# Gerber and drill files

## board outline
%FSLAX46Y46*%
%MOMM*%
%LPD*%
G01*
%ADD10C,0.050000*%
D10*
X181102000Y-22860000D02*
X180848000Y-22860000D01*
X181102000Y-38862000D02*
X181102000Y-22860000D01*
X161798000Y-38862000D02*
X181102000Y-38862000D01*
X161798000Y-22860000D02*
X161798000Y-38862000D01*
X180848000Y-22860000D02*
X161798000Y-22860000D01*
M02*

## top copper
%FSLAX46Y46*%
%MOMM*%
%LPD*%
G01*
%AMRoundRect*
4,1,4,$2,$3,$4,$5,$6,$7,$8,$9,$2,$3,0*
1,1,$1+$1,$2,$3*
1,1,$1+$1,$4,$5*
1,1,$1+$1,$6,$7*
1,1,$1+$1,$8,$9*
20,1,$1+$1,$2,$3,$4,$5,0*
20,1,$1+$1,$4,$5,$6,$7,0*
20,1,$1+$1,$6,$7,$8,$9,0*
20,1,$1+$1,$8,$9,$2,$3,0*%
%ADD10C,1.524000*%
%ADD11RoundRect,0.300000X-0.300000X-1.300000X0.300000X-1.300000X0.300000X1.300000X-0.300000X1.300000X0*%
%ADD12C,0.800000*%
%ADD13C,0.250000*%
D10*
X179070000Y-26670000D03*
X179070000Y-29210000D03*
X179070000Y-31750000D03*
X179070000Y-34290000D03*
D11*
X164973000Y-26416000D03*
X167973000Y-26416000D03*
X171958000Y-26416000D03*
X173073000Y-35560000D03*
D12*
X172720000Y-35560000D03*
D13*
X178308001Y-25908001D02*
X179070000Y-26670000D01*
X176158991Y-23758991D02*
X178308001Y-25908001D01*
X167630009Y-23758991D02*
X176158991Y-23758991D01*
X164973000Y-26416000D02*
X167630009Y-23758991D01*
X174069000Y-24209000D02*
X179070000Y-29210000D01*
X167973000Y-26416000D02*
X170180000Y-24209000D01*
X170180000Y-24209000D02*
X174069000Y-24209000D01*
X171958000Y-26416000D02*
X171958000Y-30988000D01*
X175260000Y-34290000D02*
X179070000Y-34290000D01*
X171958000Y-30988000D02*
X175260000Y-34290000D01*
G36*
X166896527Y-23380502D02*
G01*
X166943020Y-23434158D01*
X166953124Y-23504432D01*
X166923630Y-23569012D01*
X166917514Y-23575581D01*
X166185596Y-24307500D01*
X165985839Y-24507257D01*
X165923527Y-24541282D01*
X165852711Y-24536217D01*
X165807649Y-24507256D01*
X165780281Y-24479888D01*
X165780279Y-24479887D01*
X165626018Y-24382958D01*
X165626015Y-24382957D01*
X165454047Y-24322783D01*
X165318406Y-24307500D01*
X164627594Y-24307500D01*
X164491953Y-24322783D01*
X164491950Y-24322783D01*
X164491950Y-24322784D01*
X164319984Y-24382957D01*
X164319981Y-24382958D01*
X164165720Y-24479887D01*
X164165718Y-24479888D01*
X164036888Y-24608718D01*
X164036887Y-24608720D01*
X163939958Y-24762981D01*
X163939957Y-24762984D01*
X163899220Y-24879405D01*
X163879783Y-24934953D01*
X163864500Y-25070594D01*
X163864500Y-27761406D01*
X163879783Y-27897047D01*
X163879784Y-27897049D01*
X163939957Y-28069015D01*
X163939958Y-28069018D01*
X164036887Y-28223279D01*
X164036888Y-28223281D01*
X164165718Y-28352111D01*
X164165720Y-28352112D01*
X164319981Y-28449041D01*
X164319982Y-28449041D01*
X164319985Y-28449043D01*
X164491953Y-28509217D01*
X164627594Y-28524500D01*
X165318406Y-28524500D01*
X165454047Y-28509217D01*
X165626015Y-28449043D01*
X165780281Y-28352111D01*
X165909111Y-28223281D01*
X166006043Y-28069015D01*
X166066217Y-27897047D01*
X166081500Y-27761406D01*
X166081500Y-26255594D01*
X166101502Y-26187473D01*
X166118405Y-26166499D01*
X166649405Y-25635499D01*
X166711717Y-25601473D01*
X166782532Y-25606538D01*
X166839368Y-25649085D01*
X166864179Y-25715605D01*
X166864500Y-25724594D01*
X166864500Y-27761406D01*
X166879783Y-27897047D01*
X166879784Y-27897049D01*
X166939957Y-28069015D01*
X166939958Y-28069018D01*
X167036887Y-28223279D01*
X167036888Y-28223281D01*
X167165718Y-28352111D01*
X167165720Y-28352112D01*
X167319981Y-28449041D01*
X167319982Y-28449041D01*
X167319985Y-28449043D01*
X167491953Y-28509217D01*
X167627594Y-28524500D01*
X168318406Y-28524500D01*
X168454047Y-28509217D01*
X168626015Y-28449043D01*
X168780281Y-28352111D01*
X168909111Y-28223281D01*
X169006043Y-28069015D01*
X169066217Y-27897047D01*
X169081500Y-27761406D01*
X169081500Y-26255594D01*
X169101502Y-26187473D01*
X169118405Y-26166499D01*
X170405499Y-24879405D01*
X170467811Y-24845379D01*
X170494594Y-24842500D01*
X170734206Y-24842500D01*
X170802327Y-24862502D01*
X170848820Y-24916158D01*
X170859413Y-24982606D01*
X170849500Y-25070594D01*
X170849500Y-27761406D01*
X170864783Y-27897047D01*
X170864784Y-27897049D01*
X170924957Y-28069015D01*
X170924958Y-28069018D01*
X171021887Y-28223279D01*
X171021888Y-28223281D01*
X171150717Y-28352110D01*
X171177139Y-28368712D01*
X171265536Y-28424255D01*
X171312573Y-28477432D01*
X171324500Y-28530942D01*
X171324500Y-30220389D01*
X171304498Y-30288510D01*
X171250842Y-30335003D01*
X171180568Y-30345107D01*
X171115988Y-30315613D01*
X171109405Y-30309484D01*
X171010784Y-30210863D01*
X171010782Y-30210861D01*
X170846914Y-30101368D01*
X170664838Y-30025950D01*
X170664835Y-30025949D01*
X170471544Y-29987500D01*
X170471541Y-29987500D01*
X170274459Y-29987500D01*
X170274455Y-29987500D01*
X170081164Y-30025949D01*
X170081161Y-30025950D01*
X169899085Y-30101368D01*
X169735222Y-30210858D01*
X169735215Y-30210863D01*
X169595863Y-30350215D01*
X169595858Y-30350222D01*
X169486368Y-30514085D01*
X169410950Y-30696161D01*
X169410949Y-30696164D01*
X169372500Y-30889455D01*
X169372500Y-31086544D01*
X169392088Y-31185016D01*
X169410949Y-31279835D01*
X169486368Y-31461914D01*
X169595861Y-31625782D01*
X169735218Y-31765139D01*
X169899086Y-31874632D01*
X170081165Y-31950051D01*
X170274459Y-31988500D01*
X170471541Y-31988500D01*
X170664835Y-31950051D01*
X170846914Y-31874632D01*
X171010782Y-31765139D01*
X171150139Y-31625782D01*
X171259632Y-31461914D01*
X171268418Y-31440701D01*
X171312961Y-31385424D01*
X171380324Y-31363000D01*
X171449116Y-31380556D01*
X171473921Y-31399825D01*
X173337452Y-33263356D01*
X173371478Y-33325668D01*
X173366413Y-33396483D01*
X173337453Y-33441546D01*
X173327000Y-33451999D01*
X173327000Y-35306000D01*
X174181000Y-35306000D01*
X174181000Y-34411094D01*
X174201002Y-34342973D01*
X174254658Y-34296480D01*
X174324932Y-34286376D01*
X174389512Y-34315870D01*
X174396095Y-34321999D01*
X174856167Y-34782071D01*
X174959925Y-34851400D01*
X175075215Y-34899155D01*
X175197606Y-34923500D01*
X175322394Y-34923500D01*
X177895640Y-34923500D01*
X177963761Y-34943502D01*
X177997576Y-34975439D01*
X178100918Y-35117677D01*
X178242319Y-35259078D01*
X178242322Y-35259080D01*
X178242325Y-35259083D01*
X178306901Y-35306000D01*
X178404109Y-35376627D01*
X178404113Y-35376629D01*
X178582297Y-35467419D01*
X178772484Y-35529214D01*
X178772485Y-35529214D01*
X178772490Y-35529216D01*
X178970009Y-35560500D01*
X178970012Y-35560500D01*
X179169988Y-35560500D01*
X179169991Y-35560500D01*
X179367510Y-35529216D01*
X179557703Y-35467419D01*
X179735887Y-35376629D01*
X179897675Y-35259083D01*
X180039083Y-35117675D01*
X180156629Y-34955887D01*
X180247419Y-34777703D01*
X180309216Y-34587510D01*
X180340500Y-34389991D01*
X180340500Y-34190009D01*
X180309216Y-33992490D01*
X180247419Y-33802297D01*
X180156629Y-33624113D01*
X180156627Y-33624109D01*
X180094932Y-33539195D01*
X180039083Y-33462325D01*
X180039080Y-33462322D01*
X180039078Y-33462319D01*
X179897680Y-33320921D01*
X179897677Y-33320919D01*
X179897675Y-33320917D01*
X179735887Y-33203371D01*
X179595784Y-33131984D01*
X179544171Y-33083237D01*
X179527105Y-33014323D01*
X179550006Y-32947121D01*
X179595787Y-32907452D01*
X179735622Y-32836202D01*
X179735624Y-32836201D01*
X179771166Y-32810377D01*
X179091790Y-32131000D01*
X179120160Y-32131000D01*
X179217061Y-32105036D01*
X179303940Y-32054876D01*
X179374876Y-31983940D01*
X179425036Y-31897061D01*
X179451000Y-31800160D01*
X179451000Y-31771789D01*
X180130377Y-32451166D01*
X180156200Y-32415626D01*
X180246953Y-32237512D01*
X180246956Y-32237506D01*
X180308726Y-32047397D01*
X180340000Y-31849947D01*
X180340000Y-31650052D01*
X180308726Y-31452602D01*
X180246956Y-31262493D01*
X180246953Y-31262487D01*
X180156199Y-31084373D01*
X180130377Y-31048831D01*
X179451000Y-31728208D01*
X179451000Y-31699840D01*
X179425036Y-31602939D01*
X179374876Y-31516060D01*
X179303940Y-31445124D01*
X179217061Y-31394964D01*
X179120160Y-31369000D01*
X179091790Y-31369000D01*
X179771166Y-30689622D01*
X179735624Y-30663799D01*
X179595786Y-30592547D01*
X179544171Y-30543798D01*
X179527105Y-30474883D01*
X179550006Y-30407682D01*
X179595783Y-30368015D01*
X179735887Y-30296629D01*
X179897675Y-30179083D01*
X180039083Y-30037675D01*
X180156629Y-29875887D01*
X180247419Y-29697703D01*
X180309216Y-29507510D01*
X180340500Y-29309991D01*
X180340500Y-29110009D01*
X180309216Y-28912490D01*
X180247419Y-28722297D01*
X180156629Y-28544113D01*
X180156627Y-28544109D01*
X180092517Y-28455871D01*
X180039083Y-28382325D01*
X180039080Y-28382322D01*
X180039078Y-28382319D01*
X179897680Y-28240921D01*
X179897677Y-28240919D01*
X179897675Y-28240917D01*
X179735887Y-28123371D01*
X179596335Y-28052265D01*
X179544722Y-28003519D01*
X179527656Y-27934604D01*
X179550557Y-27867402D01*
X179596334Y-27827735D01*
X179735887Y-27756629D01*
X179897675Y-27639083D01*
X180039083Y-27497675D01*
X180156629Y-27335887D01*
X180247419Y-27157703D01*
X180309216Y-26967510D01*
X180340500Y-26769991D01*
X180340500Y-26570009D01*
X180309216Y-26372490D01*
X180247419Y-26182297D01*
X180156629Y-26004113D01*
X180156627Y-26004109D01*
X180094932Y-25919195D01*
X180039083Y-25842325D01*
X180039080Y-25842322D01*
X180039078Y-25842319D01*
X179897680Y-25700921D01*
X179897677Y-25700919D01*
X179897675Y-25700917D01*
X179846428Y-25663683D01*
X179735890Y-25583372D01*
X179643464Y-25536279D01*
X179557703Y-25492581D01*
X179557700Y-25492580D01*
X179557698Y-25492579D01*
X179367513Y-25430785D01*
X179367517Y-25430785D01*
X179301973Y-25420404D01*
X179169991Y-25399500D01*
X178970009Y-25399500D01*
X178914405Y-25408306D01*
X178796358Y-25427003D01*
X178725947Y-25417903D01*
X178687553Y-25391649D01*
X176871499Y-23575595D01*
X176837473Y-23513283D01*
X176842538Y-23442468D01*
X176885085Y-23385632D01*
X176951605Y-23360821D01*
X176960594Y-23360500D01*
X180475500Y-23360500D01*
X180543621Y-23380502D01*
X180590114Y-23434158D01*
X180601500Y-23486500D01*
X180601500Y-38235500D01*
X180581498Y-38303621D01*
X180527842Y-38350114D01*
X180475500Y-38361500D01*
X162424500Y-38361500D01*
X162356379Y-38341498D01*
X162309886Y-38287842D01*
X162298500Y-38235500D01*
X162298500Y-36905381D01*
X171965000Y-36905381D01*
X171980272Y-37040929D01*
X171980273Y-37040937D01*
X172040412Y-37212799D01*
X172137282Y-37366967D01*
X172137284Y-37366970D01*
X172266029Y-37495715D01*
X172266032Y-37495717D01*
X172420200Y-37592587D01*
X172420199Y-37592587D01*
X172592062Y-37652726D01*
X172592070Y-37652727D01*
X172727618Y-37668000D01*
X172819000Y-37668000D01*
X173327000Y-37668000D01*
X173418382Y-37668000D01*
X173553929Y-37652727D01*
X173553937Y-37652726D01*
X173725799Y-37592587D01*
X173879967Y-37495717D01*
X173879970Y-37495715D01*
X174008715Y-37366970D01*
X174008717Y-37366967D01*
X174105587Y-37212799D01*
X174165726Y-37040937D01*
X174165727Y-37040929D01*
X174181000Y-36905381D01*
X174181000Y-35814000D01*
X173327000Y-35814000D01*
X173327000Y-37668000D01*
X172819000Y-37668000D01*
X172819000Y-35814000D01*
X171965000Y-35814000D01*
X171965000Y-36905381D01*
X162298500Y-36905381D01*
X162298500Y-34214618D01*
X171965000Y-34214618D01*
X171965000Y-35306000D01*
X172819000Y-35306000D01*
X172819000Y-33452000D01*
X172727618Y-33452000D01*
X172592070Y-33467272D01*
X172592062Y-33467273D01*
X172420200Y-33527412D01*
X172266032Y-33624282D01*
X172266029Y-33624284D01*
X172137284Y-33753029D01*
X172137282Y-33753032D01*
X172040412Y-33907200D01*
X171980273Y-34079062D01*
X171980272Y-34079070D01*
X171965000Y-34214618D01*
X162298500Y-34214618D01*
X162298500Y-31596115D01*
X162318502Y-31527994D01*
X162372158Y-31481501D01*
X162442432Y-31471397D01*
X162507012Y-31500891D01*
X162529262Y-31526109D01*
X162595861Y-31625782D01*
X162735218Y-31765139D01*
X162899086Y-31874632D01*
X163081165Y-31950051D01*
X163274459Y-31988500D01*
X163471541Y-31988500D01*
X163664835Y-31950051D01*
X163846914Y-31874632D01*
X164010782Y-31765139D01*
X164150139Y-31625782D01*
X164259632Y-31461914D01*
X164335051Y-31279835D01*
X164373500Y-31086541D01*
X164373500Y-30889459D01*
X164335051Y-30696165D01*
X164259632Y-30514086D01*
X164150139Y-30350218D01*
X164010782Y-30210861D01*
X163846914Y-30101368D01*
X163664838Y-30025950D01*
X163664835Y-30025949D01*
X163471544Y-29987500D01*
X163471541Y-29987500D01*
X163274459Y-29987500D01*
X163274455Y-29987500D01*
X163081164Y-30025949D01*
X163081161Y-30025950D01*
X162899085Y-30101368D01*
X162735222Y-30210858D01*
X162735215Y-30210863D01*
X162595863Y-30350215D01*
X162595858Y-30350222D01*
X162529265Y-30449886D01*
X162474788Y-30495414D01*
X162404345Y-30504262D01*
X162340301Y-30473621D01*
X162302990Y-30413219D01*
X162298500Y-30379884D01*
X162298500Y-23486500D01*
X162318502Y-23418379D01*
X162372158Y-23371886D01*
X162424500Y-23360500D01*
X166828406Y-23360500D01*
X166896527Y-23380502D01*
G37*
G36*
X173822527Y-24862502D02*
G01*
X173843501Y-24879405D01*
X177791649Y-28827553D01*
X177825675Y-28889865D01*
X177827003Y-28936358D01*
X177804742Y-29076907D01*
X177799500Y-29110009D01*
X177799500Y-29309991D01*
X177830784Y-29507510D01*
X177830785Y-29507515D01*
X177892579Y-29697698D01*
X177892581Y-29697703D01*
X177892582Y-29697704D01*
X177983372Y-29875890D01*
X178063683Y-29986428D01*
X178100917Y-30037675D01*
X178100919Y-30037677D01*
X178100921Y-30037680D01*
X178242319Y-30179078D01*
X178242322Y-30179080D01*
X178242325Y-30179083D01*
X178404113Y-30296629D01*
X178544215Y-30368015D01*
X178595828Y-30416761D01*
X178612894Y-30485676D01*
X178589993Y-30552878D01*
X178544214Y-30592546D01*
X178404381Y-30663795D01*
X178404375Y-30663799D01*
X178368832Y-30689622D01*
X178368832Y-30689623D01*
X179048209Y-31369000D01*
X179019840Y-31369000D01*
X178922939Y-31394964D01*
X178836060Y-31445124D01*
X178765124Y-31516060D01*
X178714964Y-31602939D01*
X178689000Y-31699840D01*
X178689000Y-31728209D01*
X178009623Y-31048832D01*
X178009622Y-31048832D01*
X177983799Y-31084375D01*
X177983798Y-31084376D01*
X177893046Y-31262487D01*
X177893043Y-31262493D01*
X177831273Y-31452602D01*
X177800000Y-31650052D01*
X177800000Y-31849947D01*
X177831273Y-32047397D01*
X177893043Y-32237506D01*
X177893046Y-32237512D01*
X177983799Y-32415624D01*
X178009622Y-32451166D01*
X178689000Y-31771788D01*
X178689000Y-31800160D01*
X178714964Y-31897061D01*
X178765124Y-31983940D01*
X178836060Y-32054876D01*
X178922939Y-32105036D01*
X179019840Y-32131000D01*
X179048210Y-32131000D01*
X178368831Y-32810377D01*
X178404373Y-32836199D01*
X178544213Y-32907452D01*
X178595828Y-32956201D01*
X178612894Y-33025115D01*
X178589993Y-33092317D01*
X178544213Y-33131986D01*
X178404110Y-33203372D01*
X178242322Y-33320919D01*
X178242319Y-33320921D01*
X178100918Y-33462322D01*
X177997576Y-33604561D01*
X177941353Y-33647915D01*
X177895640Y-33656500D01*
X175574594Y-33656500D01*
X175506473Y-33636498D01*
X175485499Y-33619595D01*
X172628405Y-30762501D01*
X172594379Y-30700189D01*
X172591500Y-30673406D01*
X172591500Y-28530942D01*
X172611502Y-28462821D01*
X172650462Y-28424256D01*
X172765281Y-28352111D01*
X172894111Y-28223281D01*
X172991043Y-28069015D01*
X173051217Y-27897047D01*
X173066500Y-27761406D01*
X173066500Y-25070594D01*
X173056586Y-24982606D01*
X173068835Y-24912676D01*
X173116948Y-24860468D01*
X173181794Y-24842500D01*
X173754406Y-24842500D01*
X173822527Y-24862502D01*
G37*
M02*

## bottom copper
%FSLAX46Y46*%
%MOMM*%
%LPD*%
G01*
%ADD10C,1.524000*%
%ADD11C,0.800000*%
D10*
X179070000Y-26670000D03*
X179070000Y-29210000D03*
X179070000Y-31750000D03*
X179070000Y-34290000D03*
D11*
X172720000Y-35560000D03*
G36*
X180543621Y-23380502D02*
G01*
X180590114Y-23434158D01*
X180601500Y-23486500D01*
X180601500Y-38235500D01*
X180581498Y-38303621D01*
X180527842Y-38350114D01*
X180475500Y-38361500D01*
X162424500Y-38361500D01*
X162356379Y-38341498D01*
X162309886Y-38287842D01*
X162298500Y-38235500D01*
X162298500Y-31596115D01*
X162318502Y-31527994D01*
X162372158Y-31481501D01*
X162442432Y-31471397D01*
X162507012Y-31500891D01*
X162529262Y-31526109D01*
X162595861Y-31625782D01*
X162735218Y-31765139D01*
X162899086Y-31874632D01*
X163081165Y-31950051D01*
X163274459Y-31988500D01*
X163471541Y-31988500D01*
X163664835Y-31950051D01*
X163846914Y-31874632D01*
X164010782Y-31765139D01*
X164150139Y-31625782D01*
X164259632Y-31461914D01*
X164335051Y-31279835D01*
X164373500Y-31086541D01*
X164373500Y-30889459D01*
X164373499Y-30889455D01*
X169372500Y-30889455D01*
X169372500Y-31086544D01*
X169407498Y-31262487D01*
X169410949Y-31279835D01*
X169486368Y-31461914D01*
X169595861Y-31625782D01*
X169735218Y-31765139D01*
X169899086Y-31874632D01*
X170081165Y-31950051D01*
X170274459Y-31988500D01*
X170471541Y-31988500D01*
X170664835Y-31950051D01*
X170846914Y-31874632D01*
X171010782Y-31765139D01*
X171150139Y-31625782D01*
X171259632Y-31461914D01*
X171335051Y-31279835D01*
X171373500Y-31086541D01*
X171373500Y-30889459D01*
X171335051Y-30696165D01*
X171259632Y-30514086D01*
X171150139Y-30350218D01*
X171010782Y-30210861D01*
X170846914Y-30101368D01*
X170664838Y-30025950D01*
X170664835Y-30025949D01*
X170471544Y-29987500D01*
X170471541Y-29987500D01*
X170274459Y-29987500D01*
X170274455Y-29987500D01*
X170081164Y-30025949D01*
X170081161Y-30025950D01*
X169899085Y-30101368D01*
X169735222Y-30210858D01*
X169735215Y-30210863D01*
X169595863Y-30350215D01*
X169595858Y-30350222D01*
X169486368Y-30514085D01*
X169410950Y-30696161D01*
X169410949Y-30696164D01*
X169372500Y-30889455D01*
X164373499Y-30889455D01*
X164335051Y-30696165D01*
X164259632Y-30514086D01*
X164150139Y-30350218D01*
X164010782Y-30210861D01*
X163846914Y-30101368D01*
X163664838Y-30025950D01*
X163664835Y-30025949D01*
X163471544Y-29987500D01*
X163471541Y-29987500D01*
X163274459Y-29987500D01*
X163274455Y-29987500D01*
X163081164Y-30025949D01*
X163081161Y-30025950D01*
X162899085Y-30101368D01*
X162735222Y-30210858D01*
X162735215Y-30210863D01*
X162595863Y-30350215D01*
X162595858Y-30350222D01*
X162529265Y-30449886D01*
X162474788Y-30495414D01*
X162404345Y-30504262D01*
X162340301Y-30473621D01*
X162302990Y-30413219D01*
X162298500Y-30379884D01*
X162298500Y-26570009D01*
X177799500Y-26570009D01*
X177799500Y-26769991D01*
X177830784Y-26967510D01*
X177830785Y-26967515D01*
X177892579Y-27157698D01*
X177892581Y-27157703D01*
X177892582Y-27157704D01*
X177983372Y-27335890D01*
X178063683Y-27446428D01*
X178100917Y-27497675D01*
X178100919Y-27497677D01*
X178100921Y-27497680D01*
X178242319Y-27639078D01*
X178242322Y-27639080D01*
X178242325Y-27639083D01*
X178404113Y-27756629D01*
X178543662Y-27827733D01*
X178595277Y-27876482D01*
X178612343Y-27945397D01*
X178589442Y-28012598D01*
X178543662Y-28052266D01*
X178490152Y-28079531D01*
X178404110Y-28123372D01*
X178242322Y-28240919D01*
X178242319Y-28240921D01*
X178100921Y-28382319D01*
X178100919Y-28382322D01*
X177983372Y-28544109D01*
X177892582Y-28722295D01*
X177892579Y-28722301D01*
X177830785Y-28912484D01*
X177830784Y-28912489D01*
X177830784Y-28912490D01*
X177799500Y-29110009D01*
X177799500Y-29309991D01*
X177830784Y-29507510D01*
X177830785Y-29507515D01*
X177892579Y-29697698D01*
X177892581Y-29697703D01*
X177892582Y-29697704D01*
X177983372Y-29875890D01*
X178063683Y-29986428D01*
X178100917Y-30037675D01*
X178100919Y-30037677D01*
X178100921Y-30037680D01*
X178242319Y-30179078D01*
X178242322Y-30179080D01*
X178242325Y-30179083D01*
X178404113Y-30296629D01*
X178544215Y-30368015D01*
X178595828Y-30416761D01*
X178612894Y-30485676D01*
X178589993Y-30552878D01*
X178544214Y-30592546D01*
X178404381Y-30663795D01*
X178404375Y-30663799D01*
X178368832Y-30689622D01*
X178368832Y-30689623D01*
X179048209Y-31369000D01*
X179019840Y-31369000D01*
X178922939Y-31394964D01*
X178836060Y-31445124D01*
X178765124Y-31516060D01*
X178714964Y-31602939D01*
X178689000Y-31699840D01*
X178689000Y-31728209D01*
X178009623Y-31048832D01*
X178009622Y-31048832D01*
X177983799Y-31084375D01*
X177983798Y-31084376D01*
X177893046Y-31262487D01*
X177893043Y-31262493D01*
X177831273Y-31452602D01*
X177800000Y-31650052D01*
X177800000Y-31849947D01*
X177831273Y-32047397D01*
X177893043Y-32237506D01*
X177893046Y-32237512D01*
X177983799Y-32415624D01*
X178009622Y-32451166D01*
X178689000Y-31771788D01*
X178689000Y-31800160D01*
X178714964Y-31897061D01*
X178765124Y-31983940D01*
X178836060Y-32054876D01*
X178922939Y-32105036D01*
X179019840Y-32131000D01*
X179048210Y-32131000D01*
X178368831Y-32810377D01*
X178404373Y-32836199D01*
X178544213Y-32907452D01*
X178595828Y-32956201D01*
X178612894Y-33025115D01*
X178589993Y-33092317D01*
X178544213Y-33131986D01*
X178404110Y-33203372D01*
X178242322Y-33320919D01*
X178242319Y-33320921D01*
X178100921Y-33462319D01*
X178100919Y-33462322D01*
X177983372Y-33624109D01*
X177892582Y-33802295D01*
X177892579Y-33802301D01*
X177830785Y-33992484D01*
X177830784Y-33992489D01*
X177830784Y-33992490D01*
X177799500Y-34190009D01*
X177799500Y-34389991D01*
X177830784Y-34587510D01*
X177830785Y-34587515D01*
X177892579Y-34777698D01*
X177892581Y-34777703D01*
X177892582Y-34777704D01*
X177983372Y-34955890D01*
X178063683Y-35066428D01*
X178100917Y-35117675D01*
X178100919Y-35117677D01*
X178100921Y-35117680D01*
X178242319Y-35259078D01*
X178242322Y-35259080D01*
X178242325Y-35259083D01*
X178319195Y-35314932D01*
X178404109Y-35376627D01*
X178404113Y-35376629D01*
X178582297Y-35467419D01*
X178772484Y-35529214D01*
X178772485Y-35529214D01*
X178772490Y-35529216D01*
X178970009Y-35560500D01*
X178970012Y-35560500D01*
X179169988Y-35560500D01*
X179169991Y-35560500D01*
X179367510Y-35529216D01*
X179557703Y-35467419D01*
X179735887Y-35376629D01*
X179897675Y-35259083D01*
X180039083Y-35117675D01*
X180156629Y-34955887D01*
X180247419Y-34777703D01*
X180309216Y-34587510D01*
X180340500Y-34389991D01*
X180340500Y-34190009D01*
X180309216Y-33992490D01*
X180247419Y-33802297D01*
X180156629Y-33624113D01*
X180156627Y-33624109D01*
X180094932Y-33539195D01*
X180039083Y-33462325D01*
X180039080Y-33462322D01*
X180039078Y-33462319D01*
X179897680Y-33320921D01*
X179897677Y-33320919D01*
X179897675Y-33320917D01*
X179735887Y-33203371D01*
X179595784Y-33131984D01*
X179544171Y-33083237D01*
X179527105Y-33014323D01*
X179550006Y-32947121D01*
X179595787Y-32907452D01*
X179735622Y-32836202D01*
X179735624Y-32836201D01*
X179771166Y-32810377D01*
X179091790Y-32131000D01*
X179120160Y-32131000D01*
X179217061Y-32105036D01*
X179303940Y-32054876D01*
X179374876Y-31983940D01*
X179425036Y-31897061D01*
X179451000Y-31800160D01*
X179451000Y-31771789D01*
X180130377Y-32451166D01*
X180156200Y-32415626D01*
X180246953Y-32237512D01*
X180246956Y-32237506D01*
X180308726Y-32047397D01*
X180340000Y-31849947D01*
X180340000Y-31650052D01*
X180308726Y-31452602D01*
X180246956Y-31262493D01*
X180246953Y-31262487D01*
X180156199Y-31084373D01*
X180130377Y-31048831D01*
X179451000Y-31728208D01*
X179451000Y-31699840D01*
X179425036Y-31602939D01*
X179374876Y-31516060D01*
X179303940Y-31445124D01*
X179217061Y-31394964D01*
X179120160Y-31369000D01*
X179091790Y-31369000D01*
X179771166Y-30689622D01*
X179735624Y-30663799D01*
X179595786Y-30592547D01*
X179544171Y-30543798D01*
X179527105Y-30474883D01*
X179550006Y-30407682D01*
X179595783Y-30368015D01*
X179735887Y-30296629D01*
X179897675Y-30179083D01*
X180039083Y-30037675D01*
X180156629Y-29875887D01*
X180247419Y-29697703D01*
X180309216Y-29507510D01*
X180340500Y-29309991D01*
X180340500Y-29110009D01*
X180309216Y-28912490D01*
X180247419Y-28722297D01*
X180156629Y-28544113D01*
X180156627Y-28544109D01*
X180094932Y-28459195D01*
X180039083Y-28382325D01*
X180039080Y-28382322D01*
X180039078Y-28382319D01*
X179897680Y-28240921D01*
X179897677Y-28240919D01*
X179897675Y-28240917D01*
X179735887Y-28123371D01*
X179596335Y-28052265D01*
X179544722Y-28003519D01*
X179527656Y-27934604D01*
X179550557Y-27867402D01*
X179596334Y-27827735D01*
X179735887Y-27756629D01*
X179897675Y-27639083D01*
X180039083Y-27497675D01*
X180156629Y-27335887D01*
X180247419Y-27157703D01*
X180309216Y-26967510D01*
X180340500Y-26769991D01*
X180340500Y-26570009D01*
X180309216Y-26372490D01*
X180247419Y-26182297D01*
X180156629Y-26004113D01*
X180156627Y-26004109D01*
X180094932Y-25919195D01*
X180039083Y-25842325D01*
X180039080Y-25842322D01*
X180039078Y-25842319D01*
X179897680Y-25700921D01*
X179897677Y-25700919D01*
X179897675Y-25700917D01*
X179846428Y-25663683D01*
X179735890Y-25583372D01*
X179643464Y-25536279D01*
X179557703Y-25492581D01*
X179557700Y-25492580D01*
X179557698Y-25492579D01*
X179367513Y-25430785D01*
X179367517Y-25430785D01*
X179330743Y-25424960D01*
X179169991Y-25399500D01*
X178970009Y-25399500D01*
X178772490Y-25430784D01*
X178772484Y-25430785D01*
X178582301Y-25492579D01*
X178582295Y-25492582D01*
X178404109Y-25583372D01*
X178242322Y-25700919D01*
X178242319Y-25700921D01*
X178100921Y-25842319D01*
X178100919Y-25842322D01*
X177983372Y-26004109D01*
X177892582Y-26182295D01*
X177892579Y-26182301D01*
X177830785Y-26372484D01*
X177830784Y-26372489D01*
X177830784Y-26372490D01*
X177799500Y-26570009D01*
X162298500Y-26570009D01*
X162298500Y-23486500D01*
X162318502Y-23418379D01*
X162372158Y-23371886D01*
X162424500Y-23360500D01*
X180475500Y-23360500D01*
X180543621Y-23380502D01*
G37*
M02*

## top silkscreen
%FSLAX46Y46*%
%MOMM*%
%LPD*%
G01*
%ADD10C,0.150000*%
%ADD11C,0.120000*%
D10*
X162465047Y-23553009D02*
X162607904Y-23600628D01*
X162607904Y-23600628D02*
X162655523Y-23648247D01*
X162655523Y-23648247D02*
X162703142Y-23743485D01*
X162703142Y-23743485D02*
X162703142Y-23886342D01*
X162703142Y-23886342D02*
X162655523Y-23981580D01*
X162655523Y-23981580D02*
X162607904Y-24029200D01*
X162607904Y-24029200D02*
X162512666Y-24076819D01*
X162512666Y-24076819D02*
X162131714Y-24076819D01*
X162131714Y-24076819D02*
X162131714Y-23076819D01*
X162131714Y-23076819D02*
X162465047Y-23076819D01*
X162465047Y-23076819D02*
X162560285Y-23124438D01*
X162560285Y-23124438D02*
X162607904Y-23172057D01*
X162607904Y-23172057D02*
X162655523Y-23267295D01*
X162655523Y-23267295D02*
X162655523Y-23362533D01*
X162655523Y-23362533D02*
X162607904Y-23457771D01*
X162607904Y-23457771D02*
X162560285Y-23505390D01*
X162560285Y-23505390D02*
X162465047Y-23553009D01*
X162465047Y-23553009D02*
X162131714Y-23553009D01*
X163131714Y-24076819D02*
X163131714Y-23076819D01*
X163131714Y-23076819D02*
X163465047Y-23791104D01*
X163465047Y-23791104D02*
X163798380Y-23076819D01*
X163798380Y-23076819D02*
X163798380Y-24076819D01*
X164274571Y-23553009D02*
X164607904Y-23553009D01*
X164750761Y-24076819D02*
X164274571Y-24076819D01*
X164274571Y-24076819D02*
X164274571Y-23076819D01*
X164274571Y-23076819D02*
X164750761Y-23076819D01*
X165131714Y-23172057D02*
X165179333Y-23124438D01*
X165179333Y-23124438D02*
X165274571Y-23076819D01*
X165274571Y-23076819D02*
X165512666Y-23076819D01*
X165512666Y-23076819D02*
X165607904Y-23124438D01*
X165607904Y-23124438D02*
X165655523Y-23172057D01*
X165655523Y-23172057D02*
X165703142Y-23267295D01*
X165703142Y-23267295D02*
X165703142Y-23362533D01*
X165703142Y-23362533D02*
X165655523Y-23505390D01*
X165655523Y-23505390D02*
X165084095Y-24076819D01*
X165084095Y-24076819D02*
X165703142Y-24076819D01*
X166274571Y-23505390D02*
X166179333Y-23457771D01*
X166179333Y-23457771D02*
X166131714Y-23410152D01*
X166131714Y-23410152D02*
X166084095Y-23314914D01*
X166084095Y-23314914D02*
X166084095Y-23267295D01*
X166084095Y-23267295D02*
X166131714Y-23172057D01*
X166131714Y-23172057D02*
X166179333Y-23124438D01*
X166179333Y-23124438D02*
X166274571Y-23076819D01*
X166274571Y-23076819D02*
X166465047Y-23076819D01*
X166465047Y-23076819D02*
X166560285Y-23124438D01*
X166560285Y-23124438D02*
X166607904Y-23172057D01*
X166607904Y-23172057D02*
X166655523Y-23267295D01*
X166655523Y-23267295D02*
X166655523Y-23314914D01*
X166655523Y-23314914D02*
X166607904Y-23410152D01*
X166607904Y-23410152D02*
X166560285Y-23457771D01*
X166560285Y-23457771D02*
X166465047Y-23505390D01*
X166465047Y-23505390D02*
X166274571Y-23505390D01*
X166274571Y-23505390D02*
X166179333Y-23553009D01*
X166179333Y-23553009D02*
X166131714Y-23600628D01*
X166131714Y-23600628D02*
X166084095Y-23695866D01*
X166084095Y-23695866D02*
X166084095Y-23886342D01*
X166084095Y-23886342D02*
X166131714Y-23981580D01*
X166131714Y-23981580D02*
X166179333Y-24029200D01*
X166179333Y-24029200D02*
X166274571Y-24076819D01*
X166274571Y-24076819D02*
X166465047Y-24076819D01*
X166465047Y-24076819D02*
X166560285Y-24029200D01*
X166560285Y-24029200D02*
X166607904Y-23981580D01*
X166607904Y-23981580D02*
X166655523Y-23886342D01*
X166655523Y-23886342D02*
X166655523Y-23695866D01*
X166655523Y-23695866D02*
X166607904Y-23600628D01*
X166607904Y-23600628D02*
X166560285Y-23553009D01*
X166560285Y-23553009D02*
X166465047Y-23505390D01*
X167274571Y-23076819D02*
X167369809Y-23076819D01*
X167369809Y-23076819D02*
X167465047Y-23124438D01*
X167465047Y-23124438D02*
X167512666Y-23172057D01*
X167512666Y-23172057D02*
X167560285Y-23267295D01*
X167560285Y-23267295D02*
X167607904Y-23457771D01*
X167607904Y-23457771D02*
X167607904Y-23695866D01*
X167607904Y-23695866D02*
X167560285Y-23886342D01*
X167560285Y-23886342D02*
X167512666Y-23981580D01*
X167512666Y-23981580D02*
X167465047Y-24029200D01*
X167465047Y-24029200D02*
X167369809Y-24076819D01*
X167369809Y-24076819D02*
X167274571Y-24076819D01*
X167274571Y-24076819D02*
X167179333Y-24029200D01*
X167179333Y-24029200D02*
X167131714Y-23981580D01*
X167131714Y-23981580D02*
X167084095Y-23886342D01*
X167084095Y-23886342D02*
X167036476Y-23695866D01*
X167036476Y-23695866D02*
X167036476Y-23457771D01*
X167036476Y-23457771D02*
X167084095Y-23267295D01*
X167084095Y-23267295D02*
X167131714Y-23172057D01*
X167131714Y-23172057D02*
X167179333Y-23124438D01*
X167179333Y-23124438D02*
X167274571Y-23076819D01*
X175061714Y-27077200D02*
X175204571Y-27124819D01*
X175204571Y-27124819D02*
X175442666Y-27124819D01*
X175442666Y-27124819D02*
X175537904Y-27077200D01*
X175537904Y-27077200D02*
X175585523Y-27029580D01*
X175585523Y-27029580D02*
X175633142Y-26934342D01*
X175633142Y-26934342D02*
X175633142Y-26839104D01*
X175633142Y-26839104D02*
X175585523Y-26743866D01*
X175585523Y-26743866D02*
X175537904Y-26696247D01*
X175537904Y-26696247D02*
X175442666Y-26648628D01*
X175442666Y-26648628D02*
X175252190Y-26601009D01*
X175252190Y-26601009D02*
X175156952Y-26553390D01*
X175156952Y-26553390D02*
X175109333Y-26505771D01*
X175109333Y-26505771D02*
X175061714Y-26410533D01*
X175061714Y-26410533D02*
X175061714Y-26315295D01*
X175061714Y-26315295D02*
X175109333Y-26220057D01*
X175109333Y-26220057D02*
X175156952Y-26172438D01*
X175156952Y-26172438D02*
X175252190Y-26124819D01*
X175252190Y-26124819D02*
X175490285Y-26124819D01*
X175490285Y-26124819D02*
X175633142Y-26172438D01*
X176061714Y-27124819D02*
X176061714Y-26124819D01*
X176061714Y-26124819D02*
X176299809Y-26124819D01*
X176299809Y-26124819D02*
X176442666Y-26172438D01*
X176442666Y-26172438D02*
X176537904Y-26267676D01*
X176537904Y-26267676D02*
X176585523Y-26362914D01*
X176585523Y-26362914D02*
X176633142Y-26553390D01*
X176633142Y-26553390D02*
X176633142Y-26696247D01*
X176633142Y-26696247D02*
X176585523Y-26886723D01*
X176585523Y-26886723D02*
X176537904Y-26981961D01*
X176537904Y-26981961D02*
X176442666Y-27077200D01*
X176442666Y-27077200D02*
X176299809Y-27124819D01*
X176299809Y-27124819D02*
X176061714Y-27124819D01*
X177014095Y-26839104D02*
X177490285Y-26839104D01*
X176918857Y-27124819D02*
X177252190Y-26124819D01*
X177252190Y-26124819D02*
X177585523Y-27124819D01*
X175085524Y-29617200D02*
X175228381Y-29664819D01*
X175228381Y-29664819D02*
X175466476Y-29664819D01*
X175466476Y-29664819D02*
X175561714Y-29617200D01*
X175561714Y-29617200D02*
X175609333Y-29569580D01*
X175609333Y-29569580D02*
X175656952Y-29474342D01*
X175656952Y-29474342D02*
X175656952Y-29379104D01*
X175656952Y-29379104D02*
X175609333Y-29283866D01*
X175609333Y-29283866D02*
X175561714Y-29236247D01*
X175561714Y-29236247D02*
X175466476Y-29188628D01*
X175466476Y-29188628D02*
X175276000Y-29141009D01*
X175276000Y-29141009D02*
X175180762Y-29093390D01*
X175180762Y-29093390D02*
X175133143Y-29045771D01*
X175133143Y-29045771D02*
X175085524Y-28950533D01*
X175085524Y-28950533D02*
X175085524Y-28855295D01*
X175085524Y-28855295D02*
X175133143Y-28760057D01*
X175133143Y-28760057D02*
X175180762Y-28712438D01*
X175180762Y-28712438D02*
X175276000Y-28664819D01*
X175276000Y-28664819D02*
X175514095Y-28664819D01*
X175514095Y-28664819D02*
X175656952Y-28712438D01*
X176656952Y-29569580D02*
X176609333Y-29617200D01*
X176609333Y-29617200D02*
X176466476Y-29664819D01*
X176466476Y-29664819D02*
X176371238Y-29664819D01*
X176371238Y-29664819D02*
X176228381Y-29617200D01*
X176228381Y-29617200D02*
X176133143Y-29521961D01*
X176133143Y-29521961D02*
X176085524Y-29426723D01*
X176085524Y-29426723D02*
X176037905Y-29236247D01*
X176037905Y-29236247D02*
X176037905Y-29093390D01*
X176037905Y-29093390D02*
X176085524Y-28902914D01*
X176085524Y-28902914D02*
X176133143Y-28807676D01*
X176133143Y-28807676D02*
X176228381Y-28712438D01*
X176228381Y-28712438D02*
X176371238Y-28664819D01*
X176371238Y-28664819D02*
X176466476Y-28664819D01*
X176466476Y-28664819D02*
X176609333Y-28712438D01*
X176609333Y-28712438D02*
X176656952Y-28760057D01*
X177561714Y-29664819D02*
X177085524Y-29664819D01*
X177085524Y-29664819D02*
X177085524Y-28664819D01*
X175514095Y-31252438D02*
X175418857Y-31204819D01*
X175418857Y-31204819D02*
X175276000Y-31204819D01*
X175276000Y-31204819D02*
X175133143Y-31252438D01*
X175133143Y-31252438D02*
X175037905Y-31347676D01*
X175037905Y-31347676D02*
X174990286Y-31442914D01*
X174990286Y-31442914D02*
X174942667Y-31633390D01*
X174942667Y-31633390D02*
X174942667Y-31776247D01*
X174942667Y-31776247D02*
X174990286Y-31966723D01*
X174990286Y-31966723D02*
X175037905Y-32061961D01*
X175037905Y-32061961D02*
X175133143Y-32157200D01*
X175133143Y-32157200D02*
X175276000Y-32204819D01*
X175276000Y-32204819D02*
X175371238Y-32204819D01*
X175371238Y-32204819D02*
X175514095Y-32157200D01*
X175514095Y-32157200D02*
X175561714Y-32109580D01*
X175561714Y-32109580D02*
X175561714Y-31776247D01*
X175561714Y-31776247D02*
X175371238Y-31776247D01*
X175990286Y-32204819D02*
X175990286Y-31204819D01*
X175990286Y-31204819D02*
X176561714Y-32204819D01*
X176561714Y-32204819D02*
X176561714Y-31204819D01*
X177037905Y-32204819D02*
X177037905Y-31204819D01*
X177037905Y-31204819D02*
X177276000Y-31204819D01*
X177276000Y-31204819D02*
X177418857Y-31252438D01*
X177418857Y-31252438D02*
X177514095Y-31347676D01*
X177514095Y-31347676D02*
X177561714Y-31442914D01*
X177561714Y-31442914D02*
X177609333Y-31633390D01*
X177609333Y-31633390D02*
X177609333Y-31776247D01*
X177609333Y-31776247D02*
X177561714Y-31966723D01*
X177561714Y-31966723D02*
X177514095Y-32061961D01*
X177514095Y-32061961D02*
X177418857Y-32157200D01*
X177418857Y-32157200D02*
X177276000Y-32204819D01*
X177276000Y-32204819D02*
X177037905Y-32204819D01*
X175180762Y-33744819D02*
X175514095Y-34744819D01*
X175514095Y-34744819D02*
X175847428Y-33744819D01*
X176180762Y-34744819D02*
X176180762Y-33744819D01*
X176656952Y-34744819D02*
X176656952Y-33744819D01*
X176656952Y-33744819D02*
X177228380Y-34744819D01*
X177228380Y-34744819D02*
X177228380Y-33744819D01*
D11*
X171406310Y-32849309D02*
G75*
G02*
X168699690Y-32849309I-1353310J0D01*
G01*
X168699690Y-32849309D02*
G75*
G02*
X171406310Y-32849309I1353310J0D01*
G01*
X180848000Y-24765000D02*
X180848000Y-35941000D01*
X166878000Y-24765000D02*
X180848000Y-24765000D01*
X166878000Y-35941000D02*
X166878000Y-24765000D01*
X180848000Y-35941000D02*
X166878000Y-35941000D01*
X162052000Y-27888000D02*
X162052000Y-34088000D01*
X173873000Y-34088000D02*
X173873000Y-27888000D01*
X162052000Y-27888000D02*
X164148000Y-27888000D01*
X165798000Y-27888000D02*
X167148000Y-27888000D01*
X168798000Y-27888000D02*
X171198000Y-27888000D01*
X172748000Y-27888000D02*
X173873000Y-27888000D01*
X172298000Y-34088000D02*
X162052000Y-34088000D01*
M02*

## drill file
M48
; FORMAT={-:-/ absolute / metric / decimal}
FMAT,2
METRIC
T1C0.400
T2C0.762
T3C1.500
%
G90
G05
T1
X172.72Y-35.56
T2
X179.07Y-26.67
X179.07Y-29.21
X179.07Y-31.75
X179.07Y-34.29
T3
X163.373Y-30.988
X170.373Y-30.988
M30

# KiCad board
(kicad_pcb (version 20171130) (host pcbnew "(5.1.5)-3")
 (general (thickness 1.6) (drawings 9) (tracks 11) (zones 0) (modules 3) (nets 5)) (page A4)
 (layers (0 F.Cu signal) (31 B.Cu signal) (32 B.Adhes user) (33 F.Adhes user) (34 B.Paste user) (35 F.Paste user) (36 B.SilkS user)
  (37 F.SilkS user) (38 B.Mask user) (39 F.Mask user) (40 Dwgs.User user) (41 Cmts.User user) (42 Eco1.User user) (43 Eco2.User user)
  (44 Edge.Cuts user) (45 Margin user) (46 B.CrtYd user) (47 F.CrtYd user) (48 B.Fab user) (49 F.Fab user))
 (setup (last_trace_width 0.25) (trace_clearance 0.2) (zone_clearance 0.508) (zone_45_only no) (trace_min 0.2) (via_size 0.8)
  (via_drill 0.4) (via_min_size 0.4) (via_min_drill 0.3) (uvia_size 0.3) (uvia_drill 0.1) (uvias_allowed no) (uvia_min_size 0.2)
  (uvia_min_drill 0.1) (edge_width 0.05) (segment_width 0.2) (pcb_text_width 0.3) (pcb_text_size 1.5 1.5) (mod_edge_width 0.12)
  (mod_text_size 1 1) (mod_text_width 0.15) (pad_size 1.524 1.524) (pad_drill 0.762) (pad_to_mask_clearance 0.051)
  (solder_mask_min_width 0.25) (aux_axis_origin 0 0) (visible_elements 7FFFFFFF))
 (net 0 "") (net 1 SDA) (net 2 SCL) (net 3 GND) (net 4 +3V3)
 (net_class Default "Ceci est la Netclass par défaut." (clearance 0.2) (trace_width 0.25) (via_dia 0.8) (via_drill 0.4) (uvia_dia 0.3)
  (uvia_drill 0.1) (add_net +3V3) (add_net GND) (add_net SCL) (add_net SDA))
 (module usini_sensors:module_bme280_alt (layer F.Cu) (at 179.07 26.67 180)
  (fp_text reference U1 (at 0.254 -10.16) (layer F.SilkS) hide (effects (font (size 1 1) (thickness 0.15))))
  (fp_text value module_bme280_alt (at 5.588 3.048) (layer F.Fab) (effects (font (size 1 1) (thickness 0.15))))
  (fp_circle (center 9.017 -6.179309) (end 9.779 -5.060916) (layer F.SilkS) (width 0.12))
  (fp_line (start -1.778 1.905) (end -1.778 -9.271) (layer F.SilkS) (width 0.12))
  (fp_line (start 12.192 1.905) (end -1.778 1.905) (layer F.SilkS) (width 0.12))
  (fp_line (start 12.192 -9.271) (end 12.192 1.905) (layer F.SilkS) (width 0.12))
  (fp_line (start -1.778 -9.271) (end 12.192 -9.271) (layer F.SilkS) (width 0.12))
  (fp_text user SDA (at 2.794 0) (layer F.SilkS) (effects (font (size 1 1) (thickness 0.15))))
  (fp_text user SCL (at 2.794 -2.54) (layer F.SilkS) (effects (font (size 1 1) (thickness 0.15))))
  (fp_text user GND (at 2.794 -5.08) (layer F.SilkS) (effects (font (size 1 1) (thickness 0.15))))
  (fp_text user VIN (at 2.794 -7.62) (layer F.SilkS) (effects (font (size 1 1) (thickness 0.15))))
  (pad 4 thru_hole circle (at 0 0 180) (size 1.524 1.524) (drill 0.762) (layers *.Cu *.Mask) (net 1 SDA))
  (pad 3 thru_hole circle (at 0 -2.54 180) (size 1.524 1.524) (drill 0.762) (layers *.Cu *.Mask) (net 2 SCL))
  (pad 2 thru_hole circle (at 0 -5.08 180) (size 1.524 1.524) (drill 0.762) (layers *.Cu *.Mask) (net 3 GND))
  (pad 1 thru_hole circle (at 0 -7.62 180) (size 1.524 1.524) (drill 0.762) (layers *.Cu *.Mask) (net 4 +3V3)))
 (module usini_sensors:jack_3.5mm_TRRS (layer F.Cu) (at 168.148 30.988)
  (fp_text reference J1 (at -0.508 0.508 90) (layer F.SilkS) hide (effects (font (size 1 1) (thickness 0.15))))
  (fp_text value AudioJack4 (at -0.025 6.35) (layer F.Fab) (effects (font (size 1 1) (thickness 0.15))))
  (fp_line (start -6.096 -3.1) (end -6.096 3.1) (layer F.SilkS) (width 0.12))
  (fp_line (start 5.725 3.1) (end 5.725 -3.1) (layer F.SilkS) (width 0.12))
  (fp_line (start -6.096 -3.1) (end -4 -3.1) (layer F.SilkS) (width 0.12))
  (fp_line (start -2.35 -3.1) (end -1 -3.1) (layer F.SilkS) (width 0.12))
  (fp_line (start 0.65 -3.1) (end 3.05 -3.1) (layer F.SilkS) (width 0.12))
  (fp_line (start 4.6 -3.1) (end 5.725 -3.1) (layer F.SilkS) (width 0.12))
  (fp_line (start 4.15 3.1) (end -6.096 3.1) (layer F.SilkS) (width 0.12))
  (pad "" np_thru_hole circle (at 2.225 0) (size 1.5 1.5) (drill 1.5) (layers *.Cu *.Mask))
  (pad "" np_thru_hole circle (at -4.775 0) (size 1.5 1.5) (drill 1.5) (layers *.Cu *.Mask))
  (pad R2 smd roundrect (at -3.175 -4.572) (size 1.2 3.2) (layers F.Cu F.Paste F.Mask) (roundrect_rratio 0.25) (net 1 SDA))
  (pad R1 smd roundrect (at -0.175 -4.572) (size 1.2 3.2) (layers F.Cu F.Paste F.Mask) (roundrect_rratio 0.25) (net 2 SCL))
  (pad T smd roundrect (at 3.81 -4.572) (size 1.2 3.2) (layers F.Cu F.Paste F.Mask) (roundrect_rratio 0.25) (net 4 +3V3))
  (pad S smd roundrect (at 4.925 4.572) (size 1.2 3.2) (layers F.Cu F.Paste F.Mask) (roundrect_rratio 0.25) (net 3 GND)))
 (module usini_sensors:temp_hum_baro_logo (layer B.Cu) (at 173.736 35.814 180)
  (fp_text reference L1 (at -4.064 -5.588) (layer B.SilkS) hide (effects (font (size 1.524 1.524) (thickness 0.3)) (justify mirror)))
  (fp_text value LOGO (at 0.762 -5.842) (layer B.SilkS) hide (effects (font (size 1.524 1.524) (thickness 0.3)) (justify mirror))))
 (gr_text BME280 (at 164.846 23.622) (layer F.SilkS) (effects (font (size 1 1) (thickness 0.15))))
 (gr_line (start 181.102 22.86) (end 180.848 22.86) (layer Edge.Cuts) (width 0.05))
 (gr_line (start 181.102 38.862) (end 181.102 22.86) (layer Edge.Cuts) (width 0.05))
 (gr_line (start 161.798 38.862) (end 181.102 38.862) (layer Edge.Cuts) (width 0.05))
 (gr_line (start 161.798 22.86) (end 161.798 38.862) (layer Edge.Cuts) (width 0.05))
 (gr_line (start 180.848 22.86) (end 161.798 22.86) (layer Edge.Cuts) (width 0.05))
 (via (at 172.72 35.56) (size 0.8) (drill 0.4) (layers F.Cu B.Cu) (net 3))
 (segment (start 178.308001 25.908001) (end 179.07 26.67) (width 0.25) (layer F.Cu) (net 1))
 (segment (start 176.158991 23.758991) (end 178.308001 25.908001) (width 0.25) (layer F.Cu) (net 1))
 (segment (start 167.630009 23.758991) (end 176.158991 23.758991) (width 0.25) (layer F.Cu) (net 1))
 (segment (start 164.973 26.416) (end 167.630009 23.758991) (width 0.25) (layer F.Cu) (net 1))
 (segment (start 174.069 24.209) (end 179.07 29.21) (width 0.25) (layer F.Cu) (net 2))
 (segment (start 167.973 26.416) (end 170.18 24.209) (width 0.25) (layer F.Cu) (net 2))
 (segment (start 170.18 24.209) (end 174.069 24.209) (width 0.25) (layer F.Cu) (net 2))
 (segment (start 171.958 26.416) (end 171.958 30.988) (width 0.25) (layer F.Cu) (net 4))
 (segment (start 175.26 34.29) (end 179.07 34.29) (width 0.25) (layer F.Cu) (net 4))
 (segment (start 171.958 30.988) (end 175.26 34.29) (width 0.25) (layer F.Cu) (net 4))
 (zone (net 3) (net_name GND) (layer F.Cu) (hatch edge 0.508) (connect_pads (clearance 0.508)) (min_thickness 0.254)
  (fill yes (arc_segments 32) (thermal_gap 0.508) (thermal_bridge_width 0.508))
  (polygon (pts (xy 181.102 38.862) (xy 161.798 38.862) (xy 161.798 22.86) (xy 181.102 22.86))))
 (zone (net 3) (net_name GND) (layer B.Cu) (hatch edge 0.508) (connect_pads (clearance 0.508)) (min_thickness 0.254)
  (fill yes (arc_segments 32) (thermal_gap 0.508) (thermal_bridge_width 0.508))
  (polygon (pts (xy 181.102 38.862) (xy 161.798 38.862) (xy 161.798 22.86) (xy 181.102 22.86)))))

